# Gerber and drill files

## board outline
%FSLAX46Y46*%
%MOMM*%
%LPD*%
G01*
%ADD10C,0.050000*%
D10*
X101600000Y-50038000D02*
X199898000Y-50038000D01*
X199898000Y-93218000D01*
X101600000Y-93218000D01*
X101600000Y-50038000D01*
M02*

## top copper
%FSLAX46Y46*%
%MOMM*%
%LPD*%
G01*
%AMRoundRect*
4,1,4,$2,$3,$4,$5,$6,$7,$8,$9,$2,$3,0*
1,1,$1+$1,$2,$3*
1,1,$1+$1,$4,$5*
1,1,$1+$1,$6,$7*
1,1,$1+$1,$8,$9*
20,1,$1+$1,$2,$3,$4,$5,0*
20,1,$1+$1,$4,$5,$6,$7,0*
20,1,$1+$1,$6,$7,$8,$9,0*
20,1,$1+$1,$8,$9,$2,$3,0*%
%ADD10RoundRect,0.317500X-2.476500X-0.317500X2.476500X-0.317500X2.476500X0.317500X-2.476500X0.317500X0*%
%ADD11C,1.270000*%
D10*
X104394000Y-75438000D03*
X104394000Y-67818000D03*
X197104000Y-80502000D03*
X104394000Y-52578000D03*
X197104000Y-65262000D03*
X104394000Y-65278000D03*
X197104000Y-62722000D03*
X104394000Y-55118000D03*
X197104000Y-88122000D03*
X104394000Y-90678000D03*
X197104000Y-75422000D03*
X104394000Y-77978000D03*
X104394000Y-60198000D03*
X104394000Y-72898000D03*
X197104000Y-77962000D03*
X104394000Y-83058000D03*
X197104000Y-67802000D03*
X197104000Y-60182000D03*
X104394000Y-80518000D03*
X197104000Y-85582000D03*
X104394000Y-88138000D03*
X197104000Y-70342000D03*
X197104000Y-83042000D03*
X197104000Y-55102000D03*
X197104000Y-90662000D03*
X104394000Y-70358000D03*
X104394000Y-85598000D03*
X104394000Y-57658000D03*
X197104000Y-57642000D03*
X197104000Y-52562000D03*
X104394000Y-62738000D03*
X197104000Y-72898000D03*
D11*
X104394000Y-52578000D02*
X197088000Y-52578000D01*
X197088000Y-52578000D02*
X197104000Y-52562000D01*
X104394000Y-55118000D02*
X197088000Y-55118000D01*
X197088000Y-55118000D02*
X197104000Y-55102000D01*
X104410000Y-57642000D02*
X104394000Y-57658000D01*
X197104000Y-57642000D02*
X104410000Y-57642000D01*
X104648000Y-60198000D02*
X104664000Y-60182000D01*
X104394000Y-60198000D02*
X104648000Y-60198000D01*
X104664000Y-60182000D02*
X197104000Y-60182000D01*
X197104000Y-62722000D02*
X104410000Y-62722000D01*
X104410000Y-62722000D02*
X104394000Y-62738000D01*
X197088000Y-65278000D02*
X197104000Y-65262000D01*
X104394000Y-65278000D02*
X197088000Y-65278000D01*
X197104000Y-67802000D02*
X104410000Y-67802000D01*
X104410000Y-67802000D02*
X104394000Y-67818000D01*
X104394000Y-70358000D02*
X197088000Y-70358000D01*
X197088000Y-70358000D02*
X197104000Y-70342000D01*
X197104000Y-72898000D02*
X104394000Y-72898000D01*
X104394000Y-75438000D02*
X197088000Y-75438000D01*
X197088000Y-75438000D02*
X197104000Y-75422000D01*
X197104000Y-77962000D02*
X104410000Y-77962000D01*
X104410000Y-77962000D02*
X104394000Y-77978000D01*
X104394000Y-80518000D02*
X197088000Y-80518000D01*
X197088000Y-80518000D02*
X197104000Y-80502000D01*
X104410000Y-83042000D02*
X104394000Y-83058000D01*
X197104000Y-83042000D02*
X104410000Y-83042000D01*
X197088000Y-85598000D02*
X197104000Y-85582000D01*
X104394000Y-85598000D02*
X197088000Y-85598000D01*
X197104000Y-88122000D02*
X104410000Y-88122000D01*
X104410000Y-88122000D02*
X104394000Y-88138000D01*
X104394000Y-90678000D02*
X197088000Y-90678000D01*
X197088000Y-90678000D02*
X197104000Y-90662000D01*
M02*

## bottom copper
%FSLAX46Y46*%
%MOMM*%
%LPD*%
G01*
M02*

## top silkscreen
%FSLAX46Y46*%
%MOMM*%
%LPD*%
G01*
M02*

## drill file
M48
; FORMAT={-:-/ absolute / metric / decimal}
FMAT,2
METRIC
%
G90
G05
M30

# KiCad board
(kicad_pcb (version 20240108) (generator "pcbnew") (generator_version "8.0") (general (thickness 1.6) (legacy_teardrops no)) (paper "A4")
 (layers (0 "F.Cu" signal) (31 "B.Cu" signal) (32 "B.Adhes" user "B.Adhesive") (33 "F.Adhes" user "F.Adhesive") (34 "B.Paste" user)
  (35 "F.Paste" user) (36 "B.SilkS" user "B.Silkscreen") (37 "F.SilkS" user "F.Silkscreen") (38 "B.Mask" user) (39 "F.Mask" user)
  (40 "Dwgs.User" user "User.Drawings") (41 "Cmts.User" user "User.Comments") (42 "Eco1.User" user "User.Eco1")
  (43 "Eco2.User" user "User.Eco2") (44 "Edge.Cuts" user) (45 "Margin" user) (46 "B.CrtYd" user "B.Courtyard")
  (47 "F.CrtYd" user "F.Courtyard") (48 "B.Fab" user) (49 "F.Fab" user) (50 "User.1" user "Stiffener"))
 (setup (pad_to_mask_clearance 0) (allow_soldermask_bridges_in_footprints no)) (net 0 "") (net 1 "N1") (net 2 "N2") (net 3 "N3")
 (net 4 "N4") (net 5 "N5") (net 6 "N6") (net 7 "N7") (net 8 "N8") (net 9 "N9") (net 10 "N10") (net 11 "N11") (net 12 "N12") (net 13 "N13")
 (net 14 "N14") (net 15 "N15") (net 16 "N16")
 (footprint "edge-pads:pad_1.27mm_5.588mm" (layer "F.Cu") (at 104.14 75.565)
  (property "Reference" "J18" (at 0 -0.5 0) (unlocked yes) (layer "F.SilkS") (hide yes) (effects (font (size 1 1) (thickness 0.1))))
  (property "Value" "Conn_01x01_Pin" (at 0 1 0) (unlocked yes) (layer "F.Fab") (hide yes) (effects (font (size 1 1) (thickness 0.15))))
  (pad "1" smd roundrect (at 0.254 -0.127) (size 5.588 1.27) (layers "F.Cu" "F.Paste" "F.Mask") (roundrect_rratio 0.25) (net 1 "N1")
   (thermal_bridge_angle 45)))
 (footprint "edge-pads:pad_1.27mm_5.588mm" (layer "F.Cu") (at 104.14 67.945)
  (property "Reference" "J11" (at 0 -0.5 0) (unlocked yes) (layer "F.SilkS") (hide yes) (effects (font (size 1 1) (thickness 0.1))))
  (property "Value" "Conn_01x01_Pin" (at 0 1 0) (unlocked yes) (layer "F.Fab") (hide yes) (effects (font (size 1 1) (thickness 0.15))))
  (pad "1" smd roundrect (at 0.254 -0.127) (size 5.588 1.27) (layers "F.Cu" "F.Paste" "F.Mask") (roundrect_rratio 0.25) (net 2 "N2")
   (thermal_bridge_angle 45)))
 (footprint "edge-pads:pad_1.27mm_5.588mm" (layer "F.Cu") (at 196.85 80.629)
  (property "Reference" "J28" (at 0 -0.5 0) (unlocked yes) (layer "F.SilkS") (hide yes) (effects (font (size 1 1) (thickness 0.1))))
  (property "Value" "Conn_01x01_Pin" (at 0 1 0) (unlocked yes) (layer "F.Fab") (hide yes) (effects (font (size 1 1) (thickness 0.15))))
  (pad "1" smd roundrect (at 0.254 -0.127) (size 5.588 1.27) (layers "F.Cu" "F.Paste" "F.Mask") (roundrect_rratio 0.25) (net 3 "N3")
   (thermal_bridge_angle 45)))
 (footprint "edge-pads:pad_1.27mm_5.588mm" (layer "F.Cu") (at 104.14 52.705)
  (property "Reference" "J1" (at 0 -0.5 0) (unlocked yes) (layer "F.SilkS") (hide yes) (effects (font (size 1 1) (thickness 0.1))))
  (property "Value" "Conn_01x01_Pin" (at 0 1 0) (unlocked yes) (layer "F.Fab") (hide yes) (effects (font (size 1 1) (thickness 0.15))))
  (pad "1" smd roundrect (at 0.254 -0.127) (size 5.588 1.27) (layers "F.Cu" "F.Paste" "F.Mask") (roundrect_rratio 0.25) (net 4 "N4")
   (thermal_bridge_angle 45)))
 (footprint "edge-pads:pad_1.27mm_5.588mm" (layer "F.Cu") (at 196.85 65.389)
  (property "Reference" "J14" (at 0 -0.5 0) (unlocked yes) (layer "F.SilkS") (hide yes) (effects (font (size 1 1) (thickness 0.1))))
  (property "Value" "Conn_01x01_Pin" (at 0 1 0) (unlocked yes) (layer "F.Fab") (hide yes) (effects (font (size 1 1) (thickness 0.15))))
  (pad "1" smd roundrect (at 0.254 -0.127) (size 5.588 1.27) (layers "F.Cu" "F.Paste" "F.Mask") (roundrect_rratio 0.25) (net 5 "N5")
   (thermal_bridge_angle 45)))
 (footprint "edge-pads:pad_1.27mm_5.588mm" (layer "F.Cu") (at 104.14 65.405)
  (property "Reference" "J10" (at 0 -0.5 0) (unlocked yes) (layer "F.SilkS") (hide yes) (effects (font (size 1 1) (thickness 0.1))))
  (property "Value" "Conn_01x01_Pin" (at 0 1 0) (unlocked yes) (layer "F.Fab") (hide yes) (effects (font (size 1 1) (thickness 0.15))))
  (pad "1" smd roundrect (at 0.254 -0.127) (size 5.588 1.27) (layers "F.Cu" "F.Paste" "F.Mask") (roundrect_rratio 0.25) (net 5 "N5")
   (thermal_bridge_angle 45)))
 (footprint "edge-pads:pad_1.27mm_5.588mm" (layer "F.Cu") (at 196.85 62.849)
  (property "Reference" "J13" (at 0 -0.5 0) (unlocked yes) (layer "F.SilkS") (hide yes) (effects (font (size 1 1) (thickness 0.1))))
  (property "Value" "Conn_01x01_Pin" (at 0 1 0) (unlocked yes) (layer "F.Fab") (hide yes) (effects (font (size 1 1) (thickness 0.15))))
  (pad "1" smd roundrect (at 0.254 -0.127) (size 5.588 1.27) (layers "F.Cu" "F.Paste" "F.Mask") (roundrect_rratio 0.25) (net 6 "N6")
   (thermal_bridge_angle 45)))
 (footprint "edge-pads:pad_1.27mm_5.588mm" (layer "F.Cu") (at 104.14 55.245)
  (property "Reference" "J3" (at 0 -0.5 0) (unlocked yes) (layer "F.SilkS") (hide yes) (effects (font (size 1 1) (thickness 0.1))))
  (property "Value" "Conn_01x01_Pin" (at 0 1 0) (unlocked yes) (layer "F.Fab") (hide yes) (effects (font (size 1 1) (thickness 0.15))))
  (pad "1" smd roundrect (at 0.254 -0.127) (size 5.588 1.27) (layers "F.Cu" "F.Paste" "F.Mask") (roundrect_rratio 0.25) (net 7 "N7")
   (thermal_bridge_angle 45)))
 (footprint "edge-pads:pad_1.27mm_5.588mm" (layer "F.Cu") (at 196.85 88.249)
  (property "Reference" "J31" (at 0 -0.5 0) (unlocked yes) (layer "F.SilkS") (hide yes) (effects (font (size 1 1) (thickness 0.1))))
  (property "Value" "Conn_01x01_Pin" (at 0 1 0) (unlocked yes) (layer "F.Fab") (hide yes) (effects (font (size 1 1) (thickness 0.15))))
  (pad "1" smd roundrect (at 0.254 -0.127) (size 5.588 1.27) (layers "F.Cu" "F.Paste" "F.Mask") (roundrect_rratio 0.25) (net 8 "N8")
   (thermal_bridge_angle 45)))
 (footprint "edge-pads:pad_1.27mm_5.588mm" (layer "F.Cu") (at 104.14 90.805)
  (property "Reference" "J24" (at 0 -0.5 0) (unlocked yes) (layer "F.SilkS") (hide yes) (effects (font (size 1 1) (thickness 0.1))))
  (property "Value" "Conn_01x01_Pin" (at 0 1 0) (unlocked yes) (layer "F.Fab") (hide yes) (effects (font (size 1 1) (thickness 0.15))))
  (pad "1" smd roundrect (at 0.254 -0.127) (size 5.588 1.27) (layers "F.Cu" "F.Paste" "F.Mask") (roundrect_rratio 0.25) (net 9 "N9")
   (thermal_bridge_angle 45)))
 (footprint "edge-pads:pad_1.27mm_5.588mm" (layer "F.Cu") (at 196.85 75.549)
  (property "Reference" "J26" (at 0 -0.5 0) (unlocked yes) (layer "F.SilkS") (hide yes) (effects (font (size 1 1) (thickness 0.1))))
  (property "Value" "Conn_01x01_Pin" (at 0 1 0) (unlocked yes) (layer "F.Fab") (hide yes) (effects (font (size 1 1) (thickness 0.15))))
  (pad "1" smd roundrect (at 0.254 -0.127) (size 5.588 1.27) (layers "F.Cu" "F.Paste" "F.Mask") (roundrect_rratio 0.25) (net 1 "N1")
   (thermal_bridge_angle 45)))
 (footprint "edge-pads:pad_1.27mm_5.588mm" (layer "F.Cu") (at 104.14 78.105)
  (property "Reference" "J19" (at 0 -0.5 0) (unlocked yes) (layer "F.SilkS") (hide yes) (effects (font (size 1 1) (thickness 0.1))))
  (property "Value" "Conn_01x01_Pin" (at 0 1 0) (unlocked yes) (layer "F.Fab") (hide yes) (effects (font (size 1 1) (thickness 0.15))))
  (pad "1" smd roundrect (at 0.254 -0.127) (size 5.588 1.27) (layers "F.Cu" "F.Paste" "F.Mask") (roundrect_rratio 0.25) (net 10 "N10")
   (thermal_bridge_angle 45)))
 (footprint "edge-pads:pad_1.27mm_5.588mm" (layer "F.Cu") (at 104.14 60.325)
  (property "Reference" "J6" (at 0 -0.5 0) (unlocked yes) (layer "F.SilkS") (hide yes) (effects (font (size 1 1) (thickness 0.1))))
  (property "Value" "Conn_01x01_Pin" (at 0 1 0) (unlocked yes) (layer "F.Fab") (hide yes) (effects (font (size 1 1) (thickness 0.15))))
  (pad "1" smd roundrect (at 0.254 -0.127) (size 5.588 1.27) (layers "F.Cu" "F.Paste" "F.Mask") (roundrect_rratio 0.25) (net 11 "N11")
   (thermal_bridge_angle 45)))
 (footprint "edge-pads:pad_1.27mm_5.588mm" (layer "F.Cu") (at 104.14 73.025)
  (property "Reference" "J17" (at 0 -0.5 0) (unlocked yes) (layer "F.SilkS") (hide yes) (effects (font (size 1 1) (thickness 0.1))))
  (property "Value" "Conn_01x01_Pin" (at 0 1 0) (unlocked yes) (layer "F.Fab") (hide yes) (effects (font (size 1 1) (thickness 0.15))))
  (pad "1" smd roundrect (at 0.254 -0.127) (size 5.588 1.27) (layers "F.Cu" "F.Paste" "F.Mask") (roundrect_rratio 0.25) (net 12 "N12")
   (thermal_bridge_angle 45)))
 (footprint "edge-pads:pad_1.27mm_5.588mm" (layer "F.Cu") (at 196.85 78.089)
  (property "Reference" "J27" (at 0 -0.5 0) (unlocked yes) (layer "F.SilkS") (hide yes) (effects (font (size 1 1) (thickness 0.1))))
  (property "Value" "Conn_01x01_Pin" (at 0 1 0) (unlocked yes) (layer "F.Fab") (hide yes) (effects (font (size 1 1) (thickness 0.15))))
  (pad "1" smd roundrect (at 0.254 -0.127) (size 5.588 1.27) (layers "F.Cu" "F.Paste" "F.Mask") (roundrect_rratio 0.25) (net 10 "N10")
   (thermal_bridge_angle 45)))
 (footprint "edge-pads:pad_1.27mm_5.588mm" (layer "F.Cu") (at 104.14 83.185)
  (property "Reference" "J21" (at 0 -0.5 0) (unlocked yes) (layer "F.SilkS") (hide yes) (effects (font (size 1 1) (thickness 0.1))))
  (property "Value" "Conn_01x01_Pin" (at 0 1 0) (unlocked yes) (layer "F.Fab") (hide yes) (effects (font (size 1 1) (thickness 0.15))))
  (pad "1" smd roundrect (at 0.254 -0.127) (size 5.588 1.27) (layers "F.Cu" "F.Paste" "F.Mask") (roundrect_rratio 0.25) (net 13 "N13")
   (thermal_bridge_angle 45)))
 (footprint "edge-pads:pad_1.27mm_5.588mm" (layer "F.Cu") (at 196.85 67.929)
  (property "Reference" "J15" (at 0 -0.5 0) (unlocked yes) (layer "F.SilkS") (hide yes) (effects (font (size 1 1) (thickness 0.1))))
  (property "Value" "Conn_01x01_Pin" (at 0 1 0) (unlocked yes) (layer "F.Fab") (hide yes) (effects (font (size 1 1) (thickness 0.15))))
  (pad "1" smd roundrect (at 0.254 -0.127) (size 5.588 1.27) (layers "F.Cu" "F.Paste" "F.Mask") (roundrect_rratio 0.25) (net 2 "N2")
   (thermal_bridge_angle 45)))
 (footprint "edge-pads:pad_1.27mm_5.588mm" (layer "F.Cu") (at 196.85 60.309)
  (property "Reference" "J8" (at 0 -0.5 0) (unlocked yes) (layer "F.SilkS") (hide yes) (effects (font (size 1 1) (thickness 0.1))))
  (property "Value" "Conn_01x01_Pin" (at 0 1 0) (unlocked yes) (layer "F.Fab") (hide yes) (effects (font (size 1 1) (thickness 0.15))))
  (pad "1" smd roundrect (at 0.254 -0.127) (size 5.588 1.27) (layers "F.Cu" "F.Paste" "F.Mask") (roundrect_rratio 0.25) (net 11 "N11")
   (thermal_bridge_angle 45)))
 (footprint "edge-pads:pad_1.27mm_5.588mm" (layer "F.Cu") (at 104.14 80.645)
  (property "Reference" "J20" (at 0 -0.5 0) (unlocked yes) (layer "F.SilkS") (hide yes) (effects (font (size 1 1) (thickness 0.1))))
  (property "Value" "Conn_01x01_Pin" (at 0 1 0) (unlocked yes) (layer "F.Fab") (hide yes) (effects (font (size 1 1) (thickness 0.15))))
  (pad "1" smd roundrect (at 0.254 -0.127) (size 5.588 1.27) (layers "F.Cu" "F.Paste" "F.Mask") (roundrect_rratio 0.25) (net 3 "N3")
   (thermal_bridge_angle 45)))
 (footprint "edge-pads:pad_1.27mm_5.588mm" (layer "F.Cu") (at 196.85 85.709)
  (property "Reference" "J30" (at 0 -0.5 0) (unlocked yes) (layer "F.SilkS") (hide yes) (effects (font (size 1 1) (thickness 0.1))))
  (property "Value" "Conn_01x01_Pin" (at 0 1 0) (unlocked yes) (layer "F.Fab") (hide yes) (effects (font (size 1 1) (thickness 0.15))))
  (pad "1" smd roundrect (at 0.254 -0.127) (size 5.588 1.27) (layers "F.Cu" "F.Paste" "F.Mask") (roundrect_rratio 0.25) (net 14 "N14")
   (thermal_bridge_angle 45)))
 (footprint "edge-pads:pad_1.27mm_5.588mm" (layer "F.Cu") (at 104.14 88.265)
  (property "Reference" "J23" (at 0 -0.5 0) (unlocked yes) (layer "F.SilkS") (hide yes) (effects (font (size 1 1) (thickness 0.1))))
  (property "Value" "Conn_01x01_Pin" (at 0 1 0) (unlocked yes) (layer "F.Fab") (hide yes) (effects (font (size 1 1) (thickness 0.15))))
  (pad "1" smd roundrect (at 0.254 -0.127) (size 5.588 1.27) (layers "F.Cu" "F.Paste" "F.Mask") (roundrect_rratio 0.25) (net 8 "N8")
   (thermal_bridge_angle 45)))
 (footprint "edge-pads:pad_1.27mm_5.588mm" (layer "F.Cu") (at 196.85 70.469)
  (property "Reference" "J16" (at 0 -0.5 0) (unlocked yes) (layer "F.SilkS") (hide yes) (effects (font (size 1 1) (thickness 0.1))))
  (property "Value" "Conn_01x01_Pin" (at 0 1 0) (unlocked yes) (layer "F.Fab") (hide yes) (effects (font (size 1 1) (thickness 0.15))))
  (pad "1" smd roundrect (at 0.254 -0.127) (size 5.588 1.27) (layers "F.Cu" "F.Paste" "F.Mask") (roundrect_rratio 0.25) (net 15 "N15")
   (thermal_bridge_angle 45)))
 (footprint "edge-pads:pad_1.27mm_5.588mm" (layer "F.Cu") (at 196.85 83.169)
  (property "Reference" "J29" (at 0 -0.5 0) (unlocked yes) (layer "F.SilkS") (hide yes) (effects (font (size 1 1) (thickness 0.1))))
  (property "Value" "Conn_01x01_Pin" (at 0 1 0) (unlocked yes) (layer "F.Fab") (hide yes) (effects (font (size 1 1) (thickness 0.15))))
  (pad "1" smd roundrect (at 0.254 -0.127) (size 5.588 1.27) (layers "F.Cu" "F.Paste" "F.Mask") (roundrect_rratio 0.25) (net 13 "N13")
   (thermal_bridge_angle 45)))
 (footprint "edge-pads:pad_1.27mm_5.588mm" (layer "F.Cu") (at 196.85 55.229)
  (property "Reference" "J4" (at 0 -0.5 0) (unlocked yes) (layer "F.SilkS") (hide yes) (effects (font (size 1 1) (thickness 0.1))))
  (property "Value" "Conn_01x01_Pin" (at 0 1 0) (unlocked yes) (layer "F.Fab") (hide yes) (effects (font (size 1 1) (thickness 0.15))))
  (pad "1" smd roundrect (at 0.254 -0.127) (size 5.588 1.27) (layers "F.Cu" "F.Paste" "F.Mask") (roundrect_rratio 0.25) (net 7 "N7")
   (thermal_bridge_angle 45)))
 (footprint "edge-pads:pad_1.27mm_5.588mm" (layer "F.Cu") (at 196.85 90.789)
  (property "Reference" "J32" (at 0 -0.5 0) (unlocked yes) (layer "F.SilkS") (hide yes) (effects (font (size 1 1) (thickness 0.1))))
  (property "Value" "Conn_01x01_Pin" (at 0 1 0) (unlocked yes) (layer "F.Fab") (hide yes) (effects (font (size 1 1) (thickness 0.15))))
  (pad "1" smd roundrect (at 0.254 -0.127) (size 5.588 1.27) (layers "F.Cu" "F.Paste" "F.Mask") (roundrect_rratio 0.25) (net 9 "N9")
   (thermal_bridge_angle 45)))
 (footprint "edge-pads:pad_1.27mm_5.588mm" (layer "F.Cu") (at 104.14 70.485)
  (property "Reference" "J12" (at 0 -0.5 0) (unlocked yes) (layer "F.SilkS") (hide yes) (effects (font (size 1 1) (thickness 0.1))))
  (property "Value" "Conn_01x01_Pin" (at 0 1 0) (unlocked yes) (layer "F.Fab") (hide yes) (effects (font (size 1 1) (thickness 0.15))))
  (pad "1" smd roundrect (at 0.254 -0.127) (size 5.588 1.27) (layers "F.Cu" "F.Paste" "F.Mask") (roundrect_rratio 0.25) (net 15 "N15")
   (thermal_bridge_angle 45)))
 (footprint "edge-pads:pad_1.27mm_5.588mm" (layer "F.Cu") (at 104.14 85.725)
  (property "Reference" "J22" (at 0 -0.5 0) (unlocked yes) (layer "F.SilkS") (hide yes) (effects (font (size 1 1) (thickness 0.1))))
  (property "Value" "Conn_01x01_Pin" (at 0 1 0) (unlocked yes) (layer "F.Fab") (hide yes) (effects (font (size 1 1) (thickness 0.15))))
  (pad "1" smd roundrect (at 0.254 -0.127) (size 5.588 1.27) (layers "F.Cu" "F.Paste" "F.Mask") (roundrect_rratio 0.25) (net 14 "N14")
   (thermal_bridge_angle 45)))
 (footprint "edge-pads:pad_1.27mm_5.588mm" (layer "F.Cu") (at 104.14 57.785)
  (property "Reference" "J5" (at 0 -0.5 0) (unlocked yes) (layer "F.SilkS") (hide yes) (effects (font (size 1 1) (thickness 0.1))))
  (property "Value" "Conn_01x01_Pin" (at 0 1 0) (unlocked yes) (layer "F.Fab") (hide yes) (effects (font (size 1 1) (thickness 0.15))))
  (pad "1" smd roundrect (at 0.254 -0.127) (size 5.588 1.27) (layers "F.Cu" "F.Paste" "F.Mask") (roundrect_rratio 0.25) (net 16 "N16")
   (thermal_bridge_angle 45)))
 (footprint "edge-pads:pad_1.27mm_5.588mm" (layer "F.Cu") (at 196.85 57.769)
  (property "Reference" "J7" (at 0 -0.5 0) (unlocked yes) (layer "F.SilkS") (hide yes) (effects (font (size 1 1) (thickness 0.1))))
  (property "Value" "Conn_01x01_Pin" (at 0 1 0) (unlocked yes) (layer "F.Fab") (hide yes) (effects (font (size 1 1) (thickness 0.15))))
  (pad "1" smd roundrect (at 0.254 -0.127) (size 5.588 1.27) (layers "F.Cu" "F.Paste" "F.Mask") (roundrect_rratio 0.25) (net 16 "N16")
   (thermal_bridge_angle 45)))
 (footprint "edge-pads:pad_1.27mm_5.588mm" (layer "F.Cu") (at 196.85 52.689)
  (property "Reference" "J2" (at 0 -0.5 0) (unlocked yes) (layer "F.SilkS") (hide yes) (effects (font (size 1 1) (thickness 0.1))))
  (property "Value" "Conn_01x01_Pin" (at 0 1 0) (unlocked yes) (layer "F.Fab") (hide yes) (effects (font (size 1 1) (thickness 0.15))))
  (pad "1" smd roundrect (at 0.254 -0.127) (size 5.588 1.27) (layers "F.Cu" "F.Paste" "F.Mask") (roundrect_rratio 0.25) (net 4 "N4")
   (thermal_bridge_angle 45)))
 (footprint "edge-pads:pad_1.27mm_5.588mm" (layer "F.Cu") (at 104.14 62.865)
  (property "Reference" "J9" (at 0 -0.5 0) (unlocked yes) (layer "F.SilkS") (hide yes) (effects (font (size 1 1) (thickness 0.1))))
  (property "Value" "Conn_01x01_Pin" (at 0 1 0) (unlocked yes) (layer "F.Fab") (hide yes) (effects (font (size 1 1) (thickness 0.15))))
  (pad "1" smd roundrect (at 0.254 -0.127) (size 5.588 1.27) (layers "F.Cu" "F.Paste" "F.Mask") (roundrect_rratio 0.25) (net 6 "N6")
   (thermal_bridge_angle 45)))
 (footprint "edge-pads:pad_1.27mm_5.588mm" (layer "F.Cu") (at 196.85 73.025)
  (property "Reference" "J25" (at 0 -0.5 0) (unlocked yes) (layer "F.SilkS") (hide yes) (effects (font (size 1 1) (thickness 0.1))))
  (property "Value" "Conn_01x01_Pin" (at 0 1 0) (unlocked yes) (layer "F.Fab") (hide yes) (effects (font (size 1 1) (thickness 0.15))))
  (pad "1" smd roundrect (at 0.254 -0.127) (size 5.588 1.27) (layers "F.Cu" "F.Paste" "F.Mask") (roundrect_rratio 0.25) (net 12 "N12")
   (thermal_bridge_angle 45)))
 (gr_rect (start 101.6 50.038) (end 199.898 93.218) (stroke (width 0.05) (type default)) (fill none) (layer "Edge.Cuts"))
 (segment (start 104.394 52.578) (end 197.088 52.578) (width 1.27) (layer "F.Cu") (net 4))
 (segment (start 197.088 52.578) (end 197.104 52.562) (width 1.27) (layer "F.Cu") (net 4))
 (segment (start 104.394 55.118) (end 197.088 55.118) (width 1.27) (layer "F.Cu") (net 7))
 (segment (start 197.088 55.118) (end 197.104 55.102) (width 1.27) (layer "F.Cu") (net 7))
 (segment (start 104.41 57.642) (end 104.394 57.658) (width 1.27) (layer "F.Cu") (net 16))
 (segment (start 197.104 57.642) (end 104.41 57.642) (width 1.27) (layer "F.Cu") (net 16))
 (segment (start 104.648 60.198) (end 104.664 60.182) (width 1.27) (layer "F.Cu") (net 11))
 (segment (start 104.394 60.198) (end 104.648 60.198) (width 1.27) (layer "F.Cu") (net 11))
 (segment (start 104.664 60.182) (end 197.104 60.182) (width 1.27) (layer "F.Cu") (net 11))
 (segment (start 197.104 62.722) (end 104.41 62.722) (width 1.27) (layer "F.Cu") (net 6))
 (segment (start 104.41 62.722) (end 104.394 62.738) (width 1.27) (layer "F.Cu") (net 6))
 (segment (start 197.088 65.278) (end 197.104 65.262) (width 1.27) (layer "F.Cu") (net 5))
 (segment (start 104.394 65.278) (end 197.088 65.278) (width 1.27) (layer "F.Cu") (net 5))
 (segment (start 197.104 67.802) (end 104.41 67.802) (width 1.27) (layer "F.Cu") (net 2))
 (segment (start 104.41 67.802) (end 104.394 67.818) (width 1.27) (layer "F.Cu") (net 2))
 (segment (start 104.394 70.358) (end 197.088 70.358) (width 1.27) (layer "F.Cu") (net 15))
 (segment (start 197.088 70.358) (end 197.104 70.342) (width 1.27) (layer "F.Cu") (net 15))
 (segment (start 197.104 72.898) (end 104.394 72.898) (width 1.27) (layer "F.Cu") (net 12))
 (segment (start 104.394 75.438) (end 197.088 75.438) (width 1.27) (layer "F.Cu") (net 1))
 (segment (start 197.088 75.438) (end 197.104 75.422) (width 1.27) (layer "F.Cu") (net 1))
 (segment (start 197.104 77.962) (end 104.41 77.962) (width 1.27) (layer "F.Cu") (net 10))
 (segment (start 104.41 77.962) (end 104.394 77.978) (width 1.27) (layer "F.Cu") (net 10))
 (segment (start 104.394 80.518) (end 197.088 80.518) (width 1.27) (layer "F.Cu") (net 3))
 (segment (start 197.088 80.518) (end 197.104 80.502) (width 1.27) (layer "F.Cu") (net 3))
 (segment (start 104.41 83.042) (end 104.394 83.058) (width 1.27) (layer "F.Cu") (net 13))
 (segment (start 197.104 83.042) (end 104.41 83.042) (width 1.27) (layer "F.Cu") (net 13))
 (segment (start 197.088 85.598) (end 197.104 85.582) (width 1.27) (layer "F.Cu") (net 14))
 (segment (start 104.394 85.598) (end 197.088 85.598) (width 1.27) (layer "F.Cu") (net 14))
 (segment (start 197.104 88.122) (end 104.41 88.122) (width 1.27) (layer "F.Cu") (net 8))
 (segment (start 104.41 88.122) (end 104.394 88.138) (width 1.27) (layer "F.Cu") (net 8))
 (segment (start 104.394 90.678) (end 197.088 90.678) (width 1.27) (layer "F.Cu") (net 9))
 (segment (start 197.088 90.678) (end 197.104 90.662) (width 1.27) (layer "F.Cu") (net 9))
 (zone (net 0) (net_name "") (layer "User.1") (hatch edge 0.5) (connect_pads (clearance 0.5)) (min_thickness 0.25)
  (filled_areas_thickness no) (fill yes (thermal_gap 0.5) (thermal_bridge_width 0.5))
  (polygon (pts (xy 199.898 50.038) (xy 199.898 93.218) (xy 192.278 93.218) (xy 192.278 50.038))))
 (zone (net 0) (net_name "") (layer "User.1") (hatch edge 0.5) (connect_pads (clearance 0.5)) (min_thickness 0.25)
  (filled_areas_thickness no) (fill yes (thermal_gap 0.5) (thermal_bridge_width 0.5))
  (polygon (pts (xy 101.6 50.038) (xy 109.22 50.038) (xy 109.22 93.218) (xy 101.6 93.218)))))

